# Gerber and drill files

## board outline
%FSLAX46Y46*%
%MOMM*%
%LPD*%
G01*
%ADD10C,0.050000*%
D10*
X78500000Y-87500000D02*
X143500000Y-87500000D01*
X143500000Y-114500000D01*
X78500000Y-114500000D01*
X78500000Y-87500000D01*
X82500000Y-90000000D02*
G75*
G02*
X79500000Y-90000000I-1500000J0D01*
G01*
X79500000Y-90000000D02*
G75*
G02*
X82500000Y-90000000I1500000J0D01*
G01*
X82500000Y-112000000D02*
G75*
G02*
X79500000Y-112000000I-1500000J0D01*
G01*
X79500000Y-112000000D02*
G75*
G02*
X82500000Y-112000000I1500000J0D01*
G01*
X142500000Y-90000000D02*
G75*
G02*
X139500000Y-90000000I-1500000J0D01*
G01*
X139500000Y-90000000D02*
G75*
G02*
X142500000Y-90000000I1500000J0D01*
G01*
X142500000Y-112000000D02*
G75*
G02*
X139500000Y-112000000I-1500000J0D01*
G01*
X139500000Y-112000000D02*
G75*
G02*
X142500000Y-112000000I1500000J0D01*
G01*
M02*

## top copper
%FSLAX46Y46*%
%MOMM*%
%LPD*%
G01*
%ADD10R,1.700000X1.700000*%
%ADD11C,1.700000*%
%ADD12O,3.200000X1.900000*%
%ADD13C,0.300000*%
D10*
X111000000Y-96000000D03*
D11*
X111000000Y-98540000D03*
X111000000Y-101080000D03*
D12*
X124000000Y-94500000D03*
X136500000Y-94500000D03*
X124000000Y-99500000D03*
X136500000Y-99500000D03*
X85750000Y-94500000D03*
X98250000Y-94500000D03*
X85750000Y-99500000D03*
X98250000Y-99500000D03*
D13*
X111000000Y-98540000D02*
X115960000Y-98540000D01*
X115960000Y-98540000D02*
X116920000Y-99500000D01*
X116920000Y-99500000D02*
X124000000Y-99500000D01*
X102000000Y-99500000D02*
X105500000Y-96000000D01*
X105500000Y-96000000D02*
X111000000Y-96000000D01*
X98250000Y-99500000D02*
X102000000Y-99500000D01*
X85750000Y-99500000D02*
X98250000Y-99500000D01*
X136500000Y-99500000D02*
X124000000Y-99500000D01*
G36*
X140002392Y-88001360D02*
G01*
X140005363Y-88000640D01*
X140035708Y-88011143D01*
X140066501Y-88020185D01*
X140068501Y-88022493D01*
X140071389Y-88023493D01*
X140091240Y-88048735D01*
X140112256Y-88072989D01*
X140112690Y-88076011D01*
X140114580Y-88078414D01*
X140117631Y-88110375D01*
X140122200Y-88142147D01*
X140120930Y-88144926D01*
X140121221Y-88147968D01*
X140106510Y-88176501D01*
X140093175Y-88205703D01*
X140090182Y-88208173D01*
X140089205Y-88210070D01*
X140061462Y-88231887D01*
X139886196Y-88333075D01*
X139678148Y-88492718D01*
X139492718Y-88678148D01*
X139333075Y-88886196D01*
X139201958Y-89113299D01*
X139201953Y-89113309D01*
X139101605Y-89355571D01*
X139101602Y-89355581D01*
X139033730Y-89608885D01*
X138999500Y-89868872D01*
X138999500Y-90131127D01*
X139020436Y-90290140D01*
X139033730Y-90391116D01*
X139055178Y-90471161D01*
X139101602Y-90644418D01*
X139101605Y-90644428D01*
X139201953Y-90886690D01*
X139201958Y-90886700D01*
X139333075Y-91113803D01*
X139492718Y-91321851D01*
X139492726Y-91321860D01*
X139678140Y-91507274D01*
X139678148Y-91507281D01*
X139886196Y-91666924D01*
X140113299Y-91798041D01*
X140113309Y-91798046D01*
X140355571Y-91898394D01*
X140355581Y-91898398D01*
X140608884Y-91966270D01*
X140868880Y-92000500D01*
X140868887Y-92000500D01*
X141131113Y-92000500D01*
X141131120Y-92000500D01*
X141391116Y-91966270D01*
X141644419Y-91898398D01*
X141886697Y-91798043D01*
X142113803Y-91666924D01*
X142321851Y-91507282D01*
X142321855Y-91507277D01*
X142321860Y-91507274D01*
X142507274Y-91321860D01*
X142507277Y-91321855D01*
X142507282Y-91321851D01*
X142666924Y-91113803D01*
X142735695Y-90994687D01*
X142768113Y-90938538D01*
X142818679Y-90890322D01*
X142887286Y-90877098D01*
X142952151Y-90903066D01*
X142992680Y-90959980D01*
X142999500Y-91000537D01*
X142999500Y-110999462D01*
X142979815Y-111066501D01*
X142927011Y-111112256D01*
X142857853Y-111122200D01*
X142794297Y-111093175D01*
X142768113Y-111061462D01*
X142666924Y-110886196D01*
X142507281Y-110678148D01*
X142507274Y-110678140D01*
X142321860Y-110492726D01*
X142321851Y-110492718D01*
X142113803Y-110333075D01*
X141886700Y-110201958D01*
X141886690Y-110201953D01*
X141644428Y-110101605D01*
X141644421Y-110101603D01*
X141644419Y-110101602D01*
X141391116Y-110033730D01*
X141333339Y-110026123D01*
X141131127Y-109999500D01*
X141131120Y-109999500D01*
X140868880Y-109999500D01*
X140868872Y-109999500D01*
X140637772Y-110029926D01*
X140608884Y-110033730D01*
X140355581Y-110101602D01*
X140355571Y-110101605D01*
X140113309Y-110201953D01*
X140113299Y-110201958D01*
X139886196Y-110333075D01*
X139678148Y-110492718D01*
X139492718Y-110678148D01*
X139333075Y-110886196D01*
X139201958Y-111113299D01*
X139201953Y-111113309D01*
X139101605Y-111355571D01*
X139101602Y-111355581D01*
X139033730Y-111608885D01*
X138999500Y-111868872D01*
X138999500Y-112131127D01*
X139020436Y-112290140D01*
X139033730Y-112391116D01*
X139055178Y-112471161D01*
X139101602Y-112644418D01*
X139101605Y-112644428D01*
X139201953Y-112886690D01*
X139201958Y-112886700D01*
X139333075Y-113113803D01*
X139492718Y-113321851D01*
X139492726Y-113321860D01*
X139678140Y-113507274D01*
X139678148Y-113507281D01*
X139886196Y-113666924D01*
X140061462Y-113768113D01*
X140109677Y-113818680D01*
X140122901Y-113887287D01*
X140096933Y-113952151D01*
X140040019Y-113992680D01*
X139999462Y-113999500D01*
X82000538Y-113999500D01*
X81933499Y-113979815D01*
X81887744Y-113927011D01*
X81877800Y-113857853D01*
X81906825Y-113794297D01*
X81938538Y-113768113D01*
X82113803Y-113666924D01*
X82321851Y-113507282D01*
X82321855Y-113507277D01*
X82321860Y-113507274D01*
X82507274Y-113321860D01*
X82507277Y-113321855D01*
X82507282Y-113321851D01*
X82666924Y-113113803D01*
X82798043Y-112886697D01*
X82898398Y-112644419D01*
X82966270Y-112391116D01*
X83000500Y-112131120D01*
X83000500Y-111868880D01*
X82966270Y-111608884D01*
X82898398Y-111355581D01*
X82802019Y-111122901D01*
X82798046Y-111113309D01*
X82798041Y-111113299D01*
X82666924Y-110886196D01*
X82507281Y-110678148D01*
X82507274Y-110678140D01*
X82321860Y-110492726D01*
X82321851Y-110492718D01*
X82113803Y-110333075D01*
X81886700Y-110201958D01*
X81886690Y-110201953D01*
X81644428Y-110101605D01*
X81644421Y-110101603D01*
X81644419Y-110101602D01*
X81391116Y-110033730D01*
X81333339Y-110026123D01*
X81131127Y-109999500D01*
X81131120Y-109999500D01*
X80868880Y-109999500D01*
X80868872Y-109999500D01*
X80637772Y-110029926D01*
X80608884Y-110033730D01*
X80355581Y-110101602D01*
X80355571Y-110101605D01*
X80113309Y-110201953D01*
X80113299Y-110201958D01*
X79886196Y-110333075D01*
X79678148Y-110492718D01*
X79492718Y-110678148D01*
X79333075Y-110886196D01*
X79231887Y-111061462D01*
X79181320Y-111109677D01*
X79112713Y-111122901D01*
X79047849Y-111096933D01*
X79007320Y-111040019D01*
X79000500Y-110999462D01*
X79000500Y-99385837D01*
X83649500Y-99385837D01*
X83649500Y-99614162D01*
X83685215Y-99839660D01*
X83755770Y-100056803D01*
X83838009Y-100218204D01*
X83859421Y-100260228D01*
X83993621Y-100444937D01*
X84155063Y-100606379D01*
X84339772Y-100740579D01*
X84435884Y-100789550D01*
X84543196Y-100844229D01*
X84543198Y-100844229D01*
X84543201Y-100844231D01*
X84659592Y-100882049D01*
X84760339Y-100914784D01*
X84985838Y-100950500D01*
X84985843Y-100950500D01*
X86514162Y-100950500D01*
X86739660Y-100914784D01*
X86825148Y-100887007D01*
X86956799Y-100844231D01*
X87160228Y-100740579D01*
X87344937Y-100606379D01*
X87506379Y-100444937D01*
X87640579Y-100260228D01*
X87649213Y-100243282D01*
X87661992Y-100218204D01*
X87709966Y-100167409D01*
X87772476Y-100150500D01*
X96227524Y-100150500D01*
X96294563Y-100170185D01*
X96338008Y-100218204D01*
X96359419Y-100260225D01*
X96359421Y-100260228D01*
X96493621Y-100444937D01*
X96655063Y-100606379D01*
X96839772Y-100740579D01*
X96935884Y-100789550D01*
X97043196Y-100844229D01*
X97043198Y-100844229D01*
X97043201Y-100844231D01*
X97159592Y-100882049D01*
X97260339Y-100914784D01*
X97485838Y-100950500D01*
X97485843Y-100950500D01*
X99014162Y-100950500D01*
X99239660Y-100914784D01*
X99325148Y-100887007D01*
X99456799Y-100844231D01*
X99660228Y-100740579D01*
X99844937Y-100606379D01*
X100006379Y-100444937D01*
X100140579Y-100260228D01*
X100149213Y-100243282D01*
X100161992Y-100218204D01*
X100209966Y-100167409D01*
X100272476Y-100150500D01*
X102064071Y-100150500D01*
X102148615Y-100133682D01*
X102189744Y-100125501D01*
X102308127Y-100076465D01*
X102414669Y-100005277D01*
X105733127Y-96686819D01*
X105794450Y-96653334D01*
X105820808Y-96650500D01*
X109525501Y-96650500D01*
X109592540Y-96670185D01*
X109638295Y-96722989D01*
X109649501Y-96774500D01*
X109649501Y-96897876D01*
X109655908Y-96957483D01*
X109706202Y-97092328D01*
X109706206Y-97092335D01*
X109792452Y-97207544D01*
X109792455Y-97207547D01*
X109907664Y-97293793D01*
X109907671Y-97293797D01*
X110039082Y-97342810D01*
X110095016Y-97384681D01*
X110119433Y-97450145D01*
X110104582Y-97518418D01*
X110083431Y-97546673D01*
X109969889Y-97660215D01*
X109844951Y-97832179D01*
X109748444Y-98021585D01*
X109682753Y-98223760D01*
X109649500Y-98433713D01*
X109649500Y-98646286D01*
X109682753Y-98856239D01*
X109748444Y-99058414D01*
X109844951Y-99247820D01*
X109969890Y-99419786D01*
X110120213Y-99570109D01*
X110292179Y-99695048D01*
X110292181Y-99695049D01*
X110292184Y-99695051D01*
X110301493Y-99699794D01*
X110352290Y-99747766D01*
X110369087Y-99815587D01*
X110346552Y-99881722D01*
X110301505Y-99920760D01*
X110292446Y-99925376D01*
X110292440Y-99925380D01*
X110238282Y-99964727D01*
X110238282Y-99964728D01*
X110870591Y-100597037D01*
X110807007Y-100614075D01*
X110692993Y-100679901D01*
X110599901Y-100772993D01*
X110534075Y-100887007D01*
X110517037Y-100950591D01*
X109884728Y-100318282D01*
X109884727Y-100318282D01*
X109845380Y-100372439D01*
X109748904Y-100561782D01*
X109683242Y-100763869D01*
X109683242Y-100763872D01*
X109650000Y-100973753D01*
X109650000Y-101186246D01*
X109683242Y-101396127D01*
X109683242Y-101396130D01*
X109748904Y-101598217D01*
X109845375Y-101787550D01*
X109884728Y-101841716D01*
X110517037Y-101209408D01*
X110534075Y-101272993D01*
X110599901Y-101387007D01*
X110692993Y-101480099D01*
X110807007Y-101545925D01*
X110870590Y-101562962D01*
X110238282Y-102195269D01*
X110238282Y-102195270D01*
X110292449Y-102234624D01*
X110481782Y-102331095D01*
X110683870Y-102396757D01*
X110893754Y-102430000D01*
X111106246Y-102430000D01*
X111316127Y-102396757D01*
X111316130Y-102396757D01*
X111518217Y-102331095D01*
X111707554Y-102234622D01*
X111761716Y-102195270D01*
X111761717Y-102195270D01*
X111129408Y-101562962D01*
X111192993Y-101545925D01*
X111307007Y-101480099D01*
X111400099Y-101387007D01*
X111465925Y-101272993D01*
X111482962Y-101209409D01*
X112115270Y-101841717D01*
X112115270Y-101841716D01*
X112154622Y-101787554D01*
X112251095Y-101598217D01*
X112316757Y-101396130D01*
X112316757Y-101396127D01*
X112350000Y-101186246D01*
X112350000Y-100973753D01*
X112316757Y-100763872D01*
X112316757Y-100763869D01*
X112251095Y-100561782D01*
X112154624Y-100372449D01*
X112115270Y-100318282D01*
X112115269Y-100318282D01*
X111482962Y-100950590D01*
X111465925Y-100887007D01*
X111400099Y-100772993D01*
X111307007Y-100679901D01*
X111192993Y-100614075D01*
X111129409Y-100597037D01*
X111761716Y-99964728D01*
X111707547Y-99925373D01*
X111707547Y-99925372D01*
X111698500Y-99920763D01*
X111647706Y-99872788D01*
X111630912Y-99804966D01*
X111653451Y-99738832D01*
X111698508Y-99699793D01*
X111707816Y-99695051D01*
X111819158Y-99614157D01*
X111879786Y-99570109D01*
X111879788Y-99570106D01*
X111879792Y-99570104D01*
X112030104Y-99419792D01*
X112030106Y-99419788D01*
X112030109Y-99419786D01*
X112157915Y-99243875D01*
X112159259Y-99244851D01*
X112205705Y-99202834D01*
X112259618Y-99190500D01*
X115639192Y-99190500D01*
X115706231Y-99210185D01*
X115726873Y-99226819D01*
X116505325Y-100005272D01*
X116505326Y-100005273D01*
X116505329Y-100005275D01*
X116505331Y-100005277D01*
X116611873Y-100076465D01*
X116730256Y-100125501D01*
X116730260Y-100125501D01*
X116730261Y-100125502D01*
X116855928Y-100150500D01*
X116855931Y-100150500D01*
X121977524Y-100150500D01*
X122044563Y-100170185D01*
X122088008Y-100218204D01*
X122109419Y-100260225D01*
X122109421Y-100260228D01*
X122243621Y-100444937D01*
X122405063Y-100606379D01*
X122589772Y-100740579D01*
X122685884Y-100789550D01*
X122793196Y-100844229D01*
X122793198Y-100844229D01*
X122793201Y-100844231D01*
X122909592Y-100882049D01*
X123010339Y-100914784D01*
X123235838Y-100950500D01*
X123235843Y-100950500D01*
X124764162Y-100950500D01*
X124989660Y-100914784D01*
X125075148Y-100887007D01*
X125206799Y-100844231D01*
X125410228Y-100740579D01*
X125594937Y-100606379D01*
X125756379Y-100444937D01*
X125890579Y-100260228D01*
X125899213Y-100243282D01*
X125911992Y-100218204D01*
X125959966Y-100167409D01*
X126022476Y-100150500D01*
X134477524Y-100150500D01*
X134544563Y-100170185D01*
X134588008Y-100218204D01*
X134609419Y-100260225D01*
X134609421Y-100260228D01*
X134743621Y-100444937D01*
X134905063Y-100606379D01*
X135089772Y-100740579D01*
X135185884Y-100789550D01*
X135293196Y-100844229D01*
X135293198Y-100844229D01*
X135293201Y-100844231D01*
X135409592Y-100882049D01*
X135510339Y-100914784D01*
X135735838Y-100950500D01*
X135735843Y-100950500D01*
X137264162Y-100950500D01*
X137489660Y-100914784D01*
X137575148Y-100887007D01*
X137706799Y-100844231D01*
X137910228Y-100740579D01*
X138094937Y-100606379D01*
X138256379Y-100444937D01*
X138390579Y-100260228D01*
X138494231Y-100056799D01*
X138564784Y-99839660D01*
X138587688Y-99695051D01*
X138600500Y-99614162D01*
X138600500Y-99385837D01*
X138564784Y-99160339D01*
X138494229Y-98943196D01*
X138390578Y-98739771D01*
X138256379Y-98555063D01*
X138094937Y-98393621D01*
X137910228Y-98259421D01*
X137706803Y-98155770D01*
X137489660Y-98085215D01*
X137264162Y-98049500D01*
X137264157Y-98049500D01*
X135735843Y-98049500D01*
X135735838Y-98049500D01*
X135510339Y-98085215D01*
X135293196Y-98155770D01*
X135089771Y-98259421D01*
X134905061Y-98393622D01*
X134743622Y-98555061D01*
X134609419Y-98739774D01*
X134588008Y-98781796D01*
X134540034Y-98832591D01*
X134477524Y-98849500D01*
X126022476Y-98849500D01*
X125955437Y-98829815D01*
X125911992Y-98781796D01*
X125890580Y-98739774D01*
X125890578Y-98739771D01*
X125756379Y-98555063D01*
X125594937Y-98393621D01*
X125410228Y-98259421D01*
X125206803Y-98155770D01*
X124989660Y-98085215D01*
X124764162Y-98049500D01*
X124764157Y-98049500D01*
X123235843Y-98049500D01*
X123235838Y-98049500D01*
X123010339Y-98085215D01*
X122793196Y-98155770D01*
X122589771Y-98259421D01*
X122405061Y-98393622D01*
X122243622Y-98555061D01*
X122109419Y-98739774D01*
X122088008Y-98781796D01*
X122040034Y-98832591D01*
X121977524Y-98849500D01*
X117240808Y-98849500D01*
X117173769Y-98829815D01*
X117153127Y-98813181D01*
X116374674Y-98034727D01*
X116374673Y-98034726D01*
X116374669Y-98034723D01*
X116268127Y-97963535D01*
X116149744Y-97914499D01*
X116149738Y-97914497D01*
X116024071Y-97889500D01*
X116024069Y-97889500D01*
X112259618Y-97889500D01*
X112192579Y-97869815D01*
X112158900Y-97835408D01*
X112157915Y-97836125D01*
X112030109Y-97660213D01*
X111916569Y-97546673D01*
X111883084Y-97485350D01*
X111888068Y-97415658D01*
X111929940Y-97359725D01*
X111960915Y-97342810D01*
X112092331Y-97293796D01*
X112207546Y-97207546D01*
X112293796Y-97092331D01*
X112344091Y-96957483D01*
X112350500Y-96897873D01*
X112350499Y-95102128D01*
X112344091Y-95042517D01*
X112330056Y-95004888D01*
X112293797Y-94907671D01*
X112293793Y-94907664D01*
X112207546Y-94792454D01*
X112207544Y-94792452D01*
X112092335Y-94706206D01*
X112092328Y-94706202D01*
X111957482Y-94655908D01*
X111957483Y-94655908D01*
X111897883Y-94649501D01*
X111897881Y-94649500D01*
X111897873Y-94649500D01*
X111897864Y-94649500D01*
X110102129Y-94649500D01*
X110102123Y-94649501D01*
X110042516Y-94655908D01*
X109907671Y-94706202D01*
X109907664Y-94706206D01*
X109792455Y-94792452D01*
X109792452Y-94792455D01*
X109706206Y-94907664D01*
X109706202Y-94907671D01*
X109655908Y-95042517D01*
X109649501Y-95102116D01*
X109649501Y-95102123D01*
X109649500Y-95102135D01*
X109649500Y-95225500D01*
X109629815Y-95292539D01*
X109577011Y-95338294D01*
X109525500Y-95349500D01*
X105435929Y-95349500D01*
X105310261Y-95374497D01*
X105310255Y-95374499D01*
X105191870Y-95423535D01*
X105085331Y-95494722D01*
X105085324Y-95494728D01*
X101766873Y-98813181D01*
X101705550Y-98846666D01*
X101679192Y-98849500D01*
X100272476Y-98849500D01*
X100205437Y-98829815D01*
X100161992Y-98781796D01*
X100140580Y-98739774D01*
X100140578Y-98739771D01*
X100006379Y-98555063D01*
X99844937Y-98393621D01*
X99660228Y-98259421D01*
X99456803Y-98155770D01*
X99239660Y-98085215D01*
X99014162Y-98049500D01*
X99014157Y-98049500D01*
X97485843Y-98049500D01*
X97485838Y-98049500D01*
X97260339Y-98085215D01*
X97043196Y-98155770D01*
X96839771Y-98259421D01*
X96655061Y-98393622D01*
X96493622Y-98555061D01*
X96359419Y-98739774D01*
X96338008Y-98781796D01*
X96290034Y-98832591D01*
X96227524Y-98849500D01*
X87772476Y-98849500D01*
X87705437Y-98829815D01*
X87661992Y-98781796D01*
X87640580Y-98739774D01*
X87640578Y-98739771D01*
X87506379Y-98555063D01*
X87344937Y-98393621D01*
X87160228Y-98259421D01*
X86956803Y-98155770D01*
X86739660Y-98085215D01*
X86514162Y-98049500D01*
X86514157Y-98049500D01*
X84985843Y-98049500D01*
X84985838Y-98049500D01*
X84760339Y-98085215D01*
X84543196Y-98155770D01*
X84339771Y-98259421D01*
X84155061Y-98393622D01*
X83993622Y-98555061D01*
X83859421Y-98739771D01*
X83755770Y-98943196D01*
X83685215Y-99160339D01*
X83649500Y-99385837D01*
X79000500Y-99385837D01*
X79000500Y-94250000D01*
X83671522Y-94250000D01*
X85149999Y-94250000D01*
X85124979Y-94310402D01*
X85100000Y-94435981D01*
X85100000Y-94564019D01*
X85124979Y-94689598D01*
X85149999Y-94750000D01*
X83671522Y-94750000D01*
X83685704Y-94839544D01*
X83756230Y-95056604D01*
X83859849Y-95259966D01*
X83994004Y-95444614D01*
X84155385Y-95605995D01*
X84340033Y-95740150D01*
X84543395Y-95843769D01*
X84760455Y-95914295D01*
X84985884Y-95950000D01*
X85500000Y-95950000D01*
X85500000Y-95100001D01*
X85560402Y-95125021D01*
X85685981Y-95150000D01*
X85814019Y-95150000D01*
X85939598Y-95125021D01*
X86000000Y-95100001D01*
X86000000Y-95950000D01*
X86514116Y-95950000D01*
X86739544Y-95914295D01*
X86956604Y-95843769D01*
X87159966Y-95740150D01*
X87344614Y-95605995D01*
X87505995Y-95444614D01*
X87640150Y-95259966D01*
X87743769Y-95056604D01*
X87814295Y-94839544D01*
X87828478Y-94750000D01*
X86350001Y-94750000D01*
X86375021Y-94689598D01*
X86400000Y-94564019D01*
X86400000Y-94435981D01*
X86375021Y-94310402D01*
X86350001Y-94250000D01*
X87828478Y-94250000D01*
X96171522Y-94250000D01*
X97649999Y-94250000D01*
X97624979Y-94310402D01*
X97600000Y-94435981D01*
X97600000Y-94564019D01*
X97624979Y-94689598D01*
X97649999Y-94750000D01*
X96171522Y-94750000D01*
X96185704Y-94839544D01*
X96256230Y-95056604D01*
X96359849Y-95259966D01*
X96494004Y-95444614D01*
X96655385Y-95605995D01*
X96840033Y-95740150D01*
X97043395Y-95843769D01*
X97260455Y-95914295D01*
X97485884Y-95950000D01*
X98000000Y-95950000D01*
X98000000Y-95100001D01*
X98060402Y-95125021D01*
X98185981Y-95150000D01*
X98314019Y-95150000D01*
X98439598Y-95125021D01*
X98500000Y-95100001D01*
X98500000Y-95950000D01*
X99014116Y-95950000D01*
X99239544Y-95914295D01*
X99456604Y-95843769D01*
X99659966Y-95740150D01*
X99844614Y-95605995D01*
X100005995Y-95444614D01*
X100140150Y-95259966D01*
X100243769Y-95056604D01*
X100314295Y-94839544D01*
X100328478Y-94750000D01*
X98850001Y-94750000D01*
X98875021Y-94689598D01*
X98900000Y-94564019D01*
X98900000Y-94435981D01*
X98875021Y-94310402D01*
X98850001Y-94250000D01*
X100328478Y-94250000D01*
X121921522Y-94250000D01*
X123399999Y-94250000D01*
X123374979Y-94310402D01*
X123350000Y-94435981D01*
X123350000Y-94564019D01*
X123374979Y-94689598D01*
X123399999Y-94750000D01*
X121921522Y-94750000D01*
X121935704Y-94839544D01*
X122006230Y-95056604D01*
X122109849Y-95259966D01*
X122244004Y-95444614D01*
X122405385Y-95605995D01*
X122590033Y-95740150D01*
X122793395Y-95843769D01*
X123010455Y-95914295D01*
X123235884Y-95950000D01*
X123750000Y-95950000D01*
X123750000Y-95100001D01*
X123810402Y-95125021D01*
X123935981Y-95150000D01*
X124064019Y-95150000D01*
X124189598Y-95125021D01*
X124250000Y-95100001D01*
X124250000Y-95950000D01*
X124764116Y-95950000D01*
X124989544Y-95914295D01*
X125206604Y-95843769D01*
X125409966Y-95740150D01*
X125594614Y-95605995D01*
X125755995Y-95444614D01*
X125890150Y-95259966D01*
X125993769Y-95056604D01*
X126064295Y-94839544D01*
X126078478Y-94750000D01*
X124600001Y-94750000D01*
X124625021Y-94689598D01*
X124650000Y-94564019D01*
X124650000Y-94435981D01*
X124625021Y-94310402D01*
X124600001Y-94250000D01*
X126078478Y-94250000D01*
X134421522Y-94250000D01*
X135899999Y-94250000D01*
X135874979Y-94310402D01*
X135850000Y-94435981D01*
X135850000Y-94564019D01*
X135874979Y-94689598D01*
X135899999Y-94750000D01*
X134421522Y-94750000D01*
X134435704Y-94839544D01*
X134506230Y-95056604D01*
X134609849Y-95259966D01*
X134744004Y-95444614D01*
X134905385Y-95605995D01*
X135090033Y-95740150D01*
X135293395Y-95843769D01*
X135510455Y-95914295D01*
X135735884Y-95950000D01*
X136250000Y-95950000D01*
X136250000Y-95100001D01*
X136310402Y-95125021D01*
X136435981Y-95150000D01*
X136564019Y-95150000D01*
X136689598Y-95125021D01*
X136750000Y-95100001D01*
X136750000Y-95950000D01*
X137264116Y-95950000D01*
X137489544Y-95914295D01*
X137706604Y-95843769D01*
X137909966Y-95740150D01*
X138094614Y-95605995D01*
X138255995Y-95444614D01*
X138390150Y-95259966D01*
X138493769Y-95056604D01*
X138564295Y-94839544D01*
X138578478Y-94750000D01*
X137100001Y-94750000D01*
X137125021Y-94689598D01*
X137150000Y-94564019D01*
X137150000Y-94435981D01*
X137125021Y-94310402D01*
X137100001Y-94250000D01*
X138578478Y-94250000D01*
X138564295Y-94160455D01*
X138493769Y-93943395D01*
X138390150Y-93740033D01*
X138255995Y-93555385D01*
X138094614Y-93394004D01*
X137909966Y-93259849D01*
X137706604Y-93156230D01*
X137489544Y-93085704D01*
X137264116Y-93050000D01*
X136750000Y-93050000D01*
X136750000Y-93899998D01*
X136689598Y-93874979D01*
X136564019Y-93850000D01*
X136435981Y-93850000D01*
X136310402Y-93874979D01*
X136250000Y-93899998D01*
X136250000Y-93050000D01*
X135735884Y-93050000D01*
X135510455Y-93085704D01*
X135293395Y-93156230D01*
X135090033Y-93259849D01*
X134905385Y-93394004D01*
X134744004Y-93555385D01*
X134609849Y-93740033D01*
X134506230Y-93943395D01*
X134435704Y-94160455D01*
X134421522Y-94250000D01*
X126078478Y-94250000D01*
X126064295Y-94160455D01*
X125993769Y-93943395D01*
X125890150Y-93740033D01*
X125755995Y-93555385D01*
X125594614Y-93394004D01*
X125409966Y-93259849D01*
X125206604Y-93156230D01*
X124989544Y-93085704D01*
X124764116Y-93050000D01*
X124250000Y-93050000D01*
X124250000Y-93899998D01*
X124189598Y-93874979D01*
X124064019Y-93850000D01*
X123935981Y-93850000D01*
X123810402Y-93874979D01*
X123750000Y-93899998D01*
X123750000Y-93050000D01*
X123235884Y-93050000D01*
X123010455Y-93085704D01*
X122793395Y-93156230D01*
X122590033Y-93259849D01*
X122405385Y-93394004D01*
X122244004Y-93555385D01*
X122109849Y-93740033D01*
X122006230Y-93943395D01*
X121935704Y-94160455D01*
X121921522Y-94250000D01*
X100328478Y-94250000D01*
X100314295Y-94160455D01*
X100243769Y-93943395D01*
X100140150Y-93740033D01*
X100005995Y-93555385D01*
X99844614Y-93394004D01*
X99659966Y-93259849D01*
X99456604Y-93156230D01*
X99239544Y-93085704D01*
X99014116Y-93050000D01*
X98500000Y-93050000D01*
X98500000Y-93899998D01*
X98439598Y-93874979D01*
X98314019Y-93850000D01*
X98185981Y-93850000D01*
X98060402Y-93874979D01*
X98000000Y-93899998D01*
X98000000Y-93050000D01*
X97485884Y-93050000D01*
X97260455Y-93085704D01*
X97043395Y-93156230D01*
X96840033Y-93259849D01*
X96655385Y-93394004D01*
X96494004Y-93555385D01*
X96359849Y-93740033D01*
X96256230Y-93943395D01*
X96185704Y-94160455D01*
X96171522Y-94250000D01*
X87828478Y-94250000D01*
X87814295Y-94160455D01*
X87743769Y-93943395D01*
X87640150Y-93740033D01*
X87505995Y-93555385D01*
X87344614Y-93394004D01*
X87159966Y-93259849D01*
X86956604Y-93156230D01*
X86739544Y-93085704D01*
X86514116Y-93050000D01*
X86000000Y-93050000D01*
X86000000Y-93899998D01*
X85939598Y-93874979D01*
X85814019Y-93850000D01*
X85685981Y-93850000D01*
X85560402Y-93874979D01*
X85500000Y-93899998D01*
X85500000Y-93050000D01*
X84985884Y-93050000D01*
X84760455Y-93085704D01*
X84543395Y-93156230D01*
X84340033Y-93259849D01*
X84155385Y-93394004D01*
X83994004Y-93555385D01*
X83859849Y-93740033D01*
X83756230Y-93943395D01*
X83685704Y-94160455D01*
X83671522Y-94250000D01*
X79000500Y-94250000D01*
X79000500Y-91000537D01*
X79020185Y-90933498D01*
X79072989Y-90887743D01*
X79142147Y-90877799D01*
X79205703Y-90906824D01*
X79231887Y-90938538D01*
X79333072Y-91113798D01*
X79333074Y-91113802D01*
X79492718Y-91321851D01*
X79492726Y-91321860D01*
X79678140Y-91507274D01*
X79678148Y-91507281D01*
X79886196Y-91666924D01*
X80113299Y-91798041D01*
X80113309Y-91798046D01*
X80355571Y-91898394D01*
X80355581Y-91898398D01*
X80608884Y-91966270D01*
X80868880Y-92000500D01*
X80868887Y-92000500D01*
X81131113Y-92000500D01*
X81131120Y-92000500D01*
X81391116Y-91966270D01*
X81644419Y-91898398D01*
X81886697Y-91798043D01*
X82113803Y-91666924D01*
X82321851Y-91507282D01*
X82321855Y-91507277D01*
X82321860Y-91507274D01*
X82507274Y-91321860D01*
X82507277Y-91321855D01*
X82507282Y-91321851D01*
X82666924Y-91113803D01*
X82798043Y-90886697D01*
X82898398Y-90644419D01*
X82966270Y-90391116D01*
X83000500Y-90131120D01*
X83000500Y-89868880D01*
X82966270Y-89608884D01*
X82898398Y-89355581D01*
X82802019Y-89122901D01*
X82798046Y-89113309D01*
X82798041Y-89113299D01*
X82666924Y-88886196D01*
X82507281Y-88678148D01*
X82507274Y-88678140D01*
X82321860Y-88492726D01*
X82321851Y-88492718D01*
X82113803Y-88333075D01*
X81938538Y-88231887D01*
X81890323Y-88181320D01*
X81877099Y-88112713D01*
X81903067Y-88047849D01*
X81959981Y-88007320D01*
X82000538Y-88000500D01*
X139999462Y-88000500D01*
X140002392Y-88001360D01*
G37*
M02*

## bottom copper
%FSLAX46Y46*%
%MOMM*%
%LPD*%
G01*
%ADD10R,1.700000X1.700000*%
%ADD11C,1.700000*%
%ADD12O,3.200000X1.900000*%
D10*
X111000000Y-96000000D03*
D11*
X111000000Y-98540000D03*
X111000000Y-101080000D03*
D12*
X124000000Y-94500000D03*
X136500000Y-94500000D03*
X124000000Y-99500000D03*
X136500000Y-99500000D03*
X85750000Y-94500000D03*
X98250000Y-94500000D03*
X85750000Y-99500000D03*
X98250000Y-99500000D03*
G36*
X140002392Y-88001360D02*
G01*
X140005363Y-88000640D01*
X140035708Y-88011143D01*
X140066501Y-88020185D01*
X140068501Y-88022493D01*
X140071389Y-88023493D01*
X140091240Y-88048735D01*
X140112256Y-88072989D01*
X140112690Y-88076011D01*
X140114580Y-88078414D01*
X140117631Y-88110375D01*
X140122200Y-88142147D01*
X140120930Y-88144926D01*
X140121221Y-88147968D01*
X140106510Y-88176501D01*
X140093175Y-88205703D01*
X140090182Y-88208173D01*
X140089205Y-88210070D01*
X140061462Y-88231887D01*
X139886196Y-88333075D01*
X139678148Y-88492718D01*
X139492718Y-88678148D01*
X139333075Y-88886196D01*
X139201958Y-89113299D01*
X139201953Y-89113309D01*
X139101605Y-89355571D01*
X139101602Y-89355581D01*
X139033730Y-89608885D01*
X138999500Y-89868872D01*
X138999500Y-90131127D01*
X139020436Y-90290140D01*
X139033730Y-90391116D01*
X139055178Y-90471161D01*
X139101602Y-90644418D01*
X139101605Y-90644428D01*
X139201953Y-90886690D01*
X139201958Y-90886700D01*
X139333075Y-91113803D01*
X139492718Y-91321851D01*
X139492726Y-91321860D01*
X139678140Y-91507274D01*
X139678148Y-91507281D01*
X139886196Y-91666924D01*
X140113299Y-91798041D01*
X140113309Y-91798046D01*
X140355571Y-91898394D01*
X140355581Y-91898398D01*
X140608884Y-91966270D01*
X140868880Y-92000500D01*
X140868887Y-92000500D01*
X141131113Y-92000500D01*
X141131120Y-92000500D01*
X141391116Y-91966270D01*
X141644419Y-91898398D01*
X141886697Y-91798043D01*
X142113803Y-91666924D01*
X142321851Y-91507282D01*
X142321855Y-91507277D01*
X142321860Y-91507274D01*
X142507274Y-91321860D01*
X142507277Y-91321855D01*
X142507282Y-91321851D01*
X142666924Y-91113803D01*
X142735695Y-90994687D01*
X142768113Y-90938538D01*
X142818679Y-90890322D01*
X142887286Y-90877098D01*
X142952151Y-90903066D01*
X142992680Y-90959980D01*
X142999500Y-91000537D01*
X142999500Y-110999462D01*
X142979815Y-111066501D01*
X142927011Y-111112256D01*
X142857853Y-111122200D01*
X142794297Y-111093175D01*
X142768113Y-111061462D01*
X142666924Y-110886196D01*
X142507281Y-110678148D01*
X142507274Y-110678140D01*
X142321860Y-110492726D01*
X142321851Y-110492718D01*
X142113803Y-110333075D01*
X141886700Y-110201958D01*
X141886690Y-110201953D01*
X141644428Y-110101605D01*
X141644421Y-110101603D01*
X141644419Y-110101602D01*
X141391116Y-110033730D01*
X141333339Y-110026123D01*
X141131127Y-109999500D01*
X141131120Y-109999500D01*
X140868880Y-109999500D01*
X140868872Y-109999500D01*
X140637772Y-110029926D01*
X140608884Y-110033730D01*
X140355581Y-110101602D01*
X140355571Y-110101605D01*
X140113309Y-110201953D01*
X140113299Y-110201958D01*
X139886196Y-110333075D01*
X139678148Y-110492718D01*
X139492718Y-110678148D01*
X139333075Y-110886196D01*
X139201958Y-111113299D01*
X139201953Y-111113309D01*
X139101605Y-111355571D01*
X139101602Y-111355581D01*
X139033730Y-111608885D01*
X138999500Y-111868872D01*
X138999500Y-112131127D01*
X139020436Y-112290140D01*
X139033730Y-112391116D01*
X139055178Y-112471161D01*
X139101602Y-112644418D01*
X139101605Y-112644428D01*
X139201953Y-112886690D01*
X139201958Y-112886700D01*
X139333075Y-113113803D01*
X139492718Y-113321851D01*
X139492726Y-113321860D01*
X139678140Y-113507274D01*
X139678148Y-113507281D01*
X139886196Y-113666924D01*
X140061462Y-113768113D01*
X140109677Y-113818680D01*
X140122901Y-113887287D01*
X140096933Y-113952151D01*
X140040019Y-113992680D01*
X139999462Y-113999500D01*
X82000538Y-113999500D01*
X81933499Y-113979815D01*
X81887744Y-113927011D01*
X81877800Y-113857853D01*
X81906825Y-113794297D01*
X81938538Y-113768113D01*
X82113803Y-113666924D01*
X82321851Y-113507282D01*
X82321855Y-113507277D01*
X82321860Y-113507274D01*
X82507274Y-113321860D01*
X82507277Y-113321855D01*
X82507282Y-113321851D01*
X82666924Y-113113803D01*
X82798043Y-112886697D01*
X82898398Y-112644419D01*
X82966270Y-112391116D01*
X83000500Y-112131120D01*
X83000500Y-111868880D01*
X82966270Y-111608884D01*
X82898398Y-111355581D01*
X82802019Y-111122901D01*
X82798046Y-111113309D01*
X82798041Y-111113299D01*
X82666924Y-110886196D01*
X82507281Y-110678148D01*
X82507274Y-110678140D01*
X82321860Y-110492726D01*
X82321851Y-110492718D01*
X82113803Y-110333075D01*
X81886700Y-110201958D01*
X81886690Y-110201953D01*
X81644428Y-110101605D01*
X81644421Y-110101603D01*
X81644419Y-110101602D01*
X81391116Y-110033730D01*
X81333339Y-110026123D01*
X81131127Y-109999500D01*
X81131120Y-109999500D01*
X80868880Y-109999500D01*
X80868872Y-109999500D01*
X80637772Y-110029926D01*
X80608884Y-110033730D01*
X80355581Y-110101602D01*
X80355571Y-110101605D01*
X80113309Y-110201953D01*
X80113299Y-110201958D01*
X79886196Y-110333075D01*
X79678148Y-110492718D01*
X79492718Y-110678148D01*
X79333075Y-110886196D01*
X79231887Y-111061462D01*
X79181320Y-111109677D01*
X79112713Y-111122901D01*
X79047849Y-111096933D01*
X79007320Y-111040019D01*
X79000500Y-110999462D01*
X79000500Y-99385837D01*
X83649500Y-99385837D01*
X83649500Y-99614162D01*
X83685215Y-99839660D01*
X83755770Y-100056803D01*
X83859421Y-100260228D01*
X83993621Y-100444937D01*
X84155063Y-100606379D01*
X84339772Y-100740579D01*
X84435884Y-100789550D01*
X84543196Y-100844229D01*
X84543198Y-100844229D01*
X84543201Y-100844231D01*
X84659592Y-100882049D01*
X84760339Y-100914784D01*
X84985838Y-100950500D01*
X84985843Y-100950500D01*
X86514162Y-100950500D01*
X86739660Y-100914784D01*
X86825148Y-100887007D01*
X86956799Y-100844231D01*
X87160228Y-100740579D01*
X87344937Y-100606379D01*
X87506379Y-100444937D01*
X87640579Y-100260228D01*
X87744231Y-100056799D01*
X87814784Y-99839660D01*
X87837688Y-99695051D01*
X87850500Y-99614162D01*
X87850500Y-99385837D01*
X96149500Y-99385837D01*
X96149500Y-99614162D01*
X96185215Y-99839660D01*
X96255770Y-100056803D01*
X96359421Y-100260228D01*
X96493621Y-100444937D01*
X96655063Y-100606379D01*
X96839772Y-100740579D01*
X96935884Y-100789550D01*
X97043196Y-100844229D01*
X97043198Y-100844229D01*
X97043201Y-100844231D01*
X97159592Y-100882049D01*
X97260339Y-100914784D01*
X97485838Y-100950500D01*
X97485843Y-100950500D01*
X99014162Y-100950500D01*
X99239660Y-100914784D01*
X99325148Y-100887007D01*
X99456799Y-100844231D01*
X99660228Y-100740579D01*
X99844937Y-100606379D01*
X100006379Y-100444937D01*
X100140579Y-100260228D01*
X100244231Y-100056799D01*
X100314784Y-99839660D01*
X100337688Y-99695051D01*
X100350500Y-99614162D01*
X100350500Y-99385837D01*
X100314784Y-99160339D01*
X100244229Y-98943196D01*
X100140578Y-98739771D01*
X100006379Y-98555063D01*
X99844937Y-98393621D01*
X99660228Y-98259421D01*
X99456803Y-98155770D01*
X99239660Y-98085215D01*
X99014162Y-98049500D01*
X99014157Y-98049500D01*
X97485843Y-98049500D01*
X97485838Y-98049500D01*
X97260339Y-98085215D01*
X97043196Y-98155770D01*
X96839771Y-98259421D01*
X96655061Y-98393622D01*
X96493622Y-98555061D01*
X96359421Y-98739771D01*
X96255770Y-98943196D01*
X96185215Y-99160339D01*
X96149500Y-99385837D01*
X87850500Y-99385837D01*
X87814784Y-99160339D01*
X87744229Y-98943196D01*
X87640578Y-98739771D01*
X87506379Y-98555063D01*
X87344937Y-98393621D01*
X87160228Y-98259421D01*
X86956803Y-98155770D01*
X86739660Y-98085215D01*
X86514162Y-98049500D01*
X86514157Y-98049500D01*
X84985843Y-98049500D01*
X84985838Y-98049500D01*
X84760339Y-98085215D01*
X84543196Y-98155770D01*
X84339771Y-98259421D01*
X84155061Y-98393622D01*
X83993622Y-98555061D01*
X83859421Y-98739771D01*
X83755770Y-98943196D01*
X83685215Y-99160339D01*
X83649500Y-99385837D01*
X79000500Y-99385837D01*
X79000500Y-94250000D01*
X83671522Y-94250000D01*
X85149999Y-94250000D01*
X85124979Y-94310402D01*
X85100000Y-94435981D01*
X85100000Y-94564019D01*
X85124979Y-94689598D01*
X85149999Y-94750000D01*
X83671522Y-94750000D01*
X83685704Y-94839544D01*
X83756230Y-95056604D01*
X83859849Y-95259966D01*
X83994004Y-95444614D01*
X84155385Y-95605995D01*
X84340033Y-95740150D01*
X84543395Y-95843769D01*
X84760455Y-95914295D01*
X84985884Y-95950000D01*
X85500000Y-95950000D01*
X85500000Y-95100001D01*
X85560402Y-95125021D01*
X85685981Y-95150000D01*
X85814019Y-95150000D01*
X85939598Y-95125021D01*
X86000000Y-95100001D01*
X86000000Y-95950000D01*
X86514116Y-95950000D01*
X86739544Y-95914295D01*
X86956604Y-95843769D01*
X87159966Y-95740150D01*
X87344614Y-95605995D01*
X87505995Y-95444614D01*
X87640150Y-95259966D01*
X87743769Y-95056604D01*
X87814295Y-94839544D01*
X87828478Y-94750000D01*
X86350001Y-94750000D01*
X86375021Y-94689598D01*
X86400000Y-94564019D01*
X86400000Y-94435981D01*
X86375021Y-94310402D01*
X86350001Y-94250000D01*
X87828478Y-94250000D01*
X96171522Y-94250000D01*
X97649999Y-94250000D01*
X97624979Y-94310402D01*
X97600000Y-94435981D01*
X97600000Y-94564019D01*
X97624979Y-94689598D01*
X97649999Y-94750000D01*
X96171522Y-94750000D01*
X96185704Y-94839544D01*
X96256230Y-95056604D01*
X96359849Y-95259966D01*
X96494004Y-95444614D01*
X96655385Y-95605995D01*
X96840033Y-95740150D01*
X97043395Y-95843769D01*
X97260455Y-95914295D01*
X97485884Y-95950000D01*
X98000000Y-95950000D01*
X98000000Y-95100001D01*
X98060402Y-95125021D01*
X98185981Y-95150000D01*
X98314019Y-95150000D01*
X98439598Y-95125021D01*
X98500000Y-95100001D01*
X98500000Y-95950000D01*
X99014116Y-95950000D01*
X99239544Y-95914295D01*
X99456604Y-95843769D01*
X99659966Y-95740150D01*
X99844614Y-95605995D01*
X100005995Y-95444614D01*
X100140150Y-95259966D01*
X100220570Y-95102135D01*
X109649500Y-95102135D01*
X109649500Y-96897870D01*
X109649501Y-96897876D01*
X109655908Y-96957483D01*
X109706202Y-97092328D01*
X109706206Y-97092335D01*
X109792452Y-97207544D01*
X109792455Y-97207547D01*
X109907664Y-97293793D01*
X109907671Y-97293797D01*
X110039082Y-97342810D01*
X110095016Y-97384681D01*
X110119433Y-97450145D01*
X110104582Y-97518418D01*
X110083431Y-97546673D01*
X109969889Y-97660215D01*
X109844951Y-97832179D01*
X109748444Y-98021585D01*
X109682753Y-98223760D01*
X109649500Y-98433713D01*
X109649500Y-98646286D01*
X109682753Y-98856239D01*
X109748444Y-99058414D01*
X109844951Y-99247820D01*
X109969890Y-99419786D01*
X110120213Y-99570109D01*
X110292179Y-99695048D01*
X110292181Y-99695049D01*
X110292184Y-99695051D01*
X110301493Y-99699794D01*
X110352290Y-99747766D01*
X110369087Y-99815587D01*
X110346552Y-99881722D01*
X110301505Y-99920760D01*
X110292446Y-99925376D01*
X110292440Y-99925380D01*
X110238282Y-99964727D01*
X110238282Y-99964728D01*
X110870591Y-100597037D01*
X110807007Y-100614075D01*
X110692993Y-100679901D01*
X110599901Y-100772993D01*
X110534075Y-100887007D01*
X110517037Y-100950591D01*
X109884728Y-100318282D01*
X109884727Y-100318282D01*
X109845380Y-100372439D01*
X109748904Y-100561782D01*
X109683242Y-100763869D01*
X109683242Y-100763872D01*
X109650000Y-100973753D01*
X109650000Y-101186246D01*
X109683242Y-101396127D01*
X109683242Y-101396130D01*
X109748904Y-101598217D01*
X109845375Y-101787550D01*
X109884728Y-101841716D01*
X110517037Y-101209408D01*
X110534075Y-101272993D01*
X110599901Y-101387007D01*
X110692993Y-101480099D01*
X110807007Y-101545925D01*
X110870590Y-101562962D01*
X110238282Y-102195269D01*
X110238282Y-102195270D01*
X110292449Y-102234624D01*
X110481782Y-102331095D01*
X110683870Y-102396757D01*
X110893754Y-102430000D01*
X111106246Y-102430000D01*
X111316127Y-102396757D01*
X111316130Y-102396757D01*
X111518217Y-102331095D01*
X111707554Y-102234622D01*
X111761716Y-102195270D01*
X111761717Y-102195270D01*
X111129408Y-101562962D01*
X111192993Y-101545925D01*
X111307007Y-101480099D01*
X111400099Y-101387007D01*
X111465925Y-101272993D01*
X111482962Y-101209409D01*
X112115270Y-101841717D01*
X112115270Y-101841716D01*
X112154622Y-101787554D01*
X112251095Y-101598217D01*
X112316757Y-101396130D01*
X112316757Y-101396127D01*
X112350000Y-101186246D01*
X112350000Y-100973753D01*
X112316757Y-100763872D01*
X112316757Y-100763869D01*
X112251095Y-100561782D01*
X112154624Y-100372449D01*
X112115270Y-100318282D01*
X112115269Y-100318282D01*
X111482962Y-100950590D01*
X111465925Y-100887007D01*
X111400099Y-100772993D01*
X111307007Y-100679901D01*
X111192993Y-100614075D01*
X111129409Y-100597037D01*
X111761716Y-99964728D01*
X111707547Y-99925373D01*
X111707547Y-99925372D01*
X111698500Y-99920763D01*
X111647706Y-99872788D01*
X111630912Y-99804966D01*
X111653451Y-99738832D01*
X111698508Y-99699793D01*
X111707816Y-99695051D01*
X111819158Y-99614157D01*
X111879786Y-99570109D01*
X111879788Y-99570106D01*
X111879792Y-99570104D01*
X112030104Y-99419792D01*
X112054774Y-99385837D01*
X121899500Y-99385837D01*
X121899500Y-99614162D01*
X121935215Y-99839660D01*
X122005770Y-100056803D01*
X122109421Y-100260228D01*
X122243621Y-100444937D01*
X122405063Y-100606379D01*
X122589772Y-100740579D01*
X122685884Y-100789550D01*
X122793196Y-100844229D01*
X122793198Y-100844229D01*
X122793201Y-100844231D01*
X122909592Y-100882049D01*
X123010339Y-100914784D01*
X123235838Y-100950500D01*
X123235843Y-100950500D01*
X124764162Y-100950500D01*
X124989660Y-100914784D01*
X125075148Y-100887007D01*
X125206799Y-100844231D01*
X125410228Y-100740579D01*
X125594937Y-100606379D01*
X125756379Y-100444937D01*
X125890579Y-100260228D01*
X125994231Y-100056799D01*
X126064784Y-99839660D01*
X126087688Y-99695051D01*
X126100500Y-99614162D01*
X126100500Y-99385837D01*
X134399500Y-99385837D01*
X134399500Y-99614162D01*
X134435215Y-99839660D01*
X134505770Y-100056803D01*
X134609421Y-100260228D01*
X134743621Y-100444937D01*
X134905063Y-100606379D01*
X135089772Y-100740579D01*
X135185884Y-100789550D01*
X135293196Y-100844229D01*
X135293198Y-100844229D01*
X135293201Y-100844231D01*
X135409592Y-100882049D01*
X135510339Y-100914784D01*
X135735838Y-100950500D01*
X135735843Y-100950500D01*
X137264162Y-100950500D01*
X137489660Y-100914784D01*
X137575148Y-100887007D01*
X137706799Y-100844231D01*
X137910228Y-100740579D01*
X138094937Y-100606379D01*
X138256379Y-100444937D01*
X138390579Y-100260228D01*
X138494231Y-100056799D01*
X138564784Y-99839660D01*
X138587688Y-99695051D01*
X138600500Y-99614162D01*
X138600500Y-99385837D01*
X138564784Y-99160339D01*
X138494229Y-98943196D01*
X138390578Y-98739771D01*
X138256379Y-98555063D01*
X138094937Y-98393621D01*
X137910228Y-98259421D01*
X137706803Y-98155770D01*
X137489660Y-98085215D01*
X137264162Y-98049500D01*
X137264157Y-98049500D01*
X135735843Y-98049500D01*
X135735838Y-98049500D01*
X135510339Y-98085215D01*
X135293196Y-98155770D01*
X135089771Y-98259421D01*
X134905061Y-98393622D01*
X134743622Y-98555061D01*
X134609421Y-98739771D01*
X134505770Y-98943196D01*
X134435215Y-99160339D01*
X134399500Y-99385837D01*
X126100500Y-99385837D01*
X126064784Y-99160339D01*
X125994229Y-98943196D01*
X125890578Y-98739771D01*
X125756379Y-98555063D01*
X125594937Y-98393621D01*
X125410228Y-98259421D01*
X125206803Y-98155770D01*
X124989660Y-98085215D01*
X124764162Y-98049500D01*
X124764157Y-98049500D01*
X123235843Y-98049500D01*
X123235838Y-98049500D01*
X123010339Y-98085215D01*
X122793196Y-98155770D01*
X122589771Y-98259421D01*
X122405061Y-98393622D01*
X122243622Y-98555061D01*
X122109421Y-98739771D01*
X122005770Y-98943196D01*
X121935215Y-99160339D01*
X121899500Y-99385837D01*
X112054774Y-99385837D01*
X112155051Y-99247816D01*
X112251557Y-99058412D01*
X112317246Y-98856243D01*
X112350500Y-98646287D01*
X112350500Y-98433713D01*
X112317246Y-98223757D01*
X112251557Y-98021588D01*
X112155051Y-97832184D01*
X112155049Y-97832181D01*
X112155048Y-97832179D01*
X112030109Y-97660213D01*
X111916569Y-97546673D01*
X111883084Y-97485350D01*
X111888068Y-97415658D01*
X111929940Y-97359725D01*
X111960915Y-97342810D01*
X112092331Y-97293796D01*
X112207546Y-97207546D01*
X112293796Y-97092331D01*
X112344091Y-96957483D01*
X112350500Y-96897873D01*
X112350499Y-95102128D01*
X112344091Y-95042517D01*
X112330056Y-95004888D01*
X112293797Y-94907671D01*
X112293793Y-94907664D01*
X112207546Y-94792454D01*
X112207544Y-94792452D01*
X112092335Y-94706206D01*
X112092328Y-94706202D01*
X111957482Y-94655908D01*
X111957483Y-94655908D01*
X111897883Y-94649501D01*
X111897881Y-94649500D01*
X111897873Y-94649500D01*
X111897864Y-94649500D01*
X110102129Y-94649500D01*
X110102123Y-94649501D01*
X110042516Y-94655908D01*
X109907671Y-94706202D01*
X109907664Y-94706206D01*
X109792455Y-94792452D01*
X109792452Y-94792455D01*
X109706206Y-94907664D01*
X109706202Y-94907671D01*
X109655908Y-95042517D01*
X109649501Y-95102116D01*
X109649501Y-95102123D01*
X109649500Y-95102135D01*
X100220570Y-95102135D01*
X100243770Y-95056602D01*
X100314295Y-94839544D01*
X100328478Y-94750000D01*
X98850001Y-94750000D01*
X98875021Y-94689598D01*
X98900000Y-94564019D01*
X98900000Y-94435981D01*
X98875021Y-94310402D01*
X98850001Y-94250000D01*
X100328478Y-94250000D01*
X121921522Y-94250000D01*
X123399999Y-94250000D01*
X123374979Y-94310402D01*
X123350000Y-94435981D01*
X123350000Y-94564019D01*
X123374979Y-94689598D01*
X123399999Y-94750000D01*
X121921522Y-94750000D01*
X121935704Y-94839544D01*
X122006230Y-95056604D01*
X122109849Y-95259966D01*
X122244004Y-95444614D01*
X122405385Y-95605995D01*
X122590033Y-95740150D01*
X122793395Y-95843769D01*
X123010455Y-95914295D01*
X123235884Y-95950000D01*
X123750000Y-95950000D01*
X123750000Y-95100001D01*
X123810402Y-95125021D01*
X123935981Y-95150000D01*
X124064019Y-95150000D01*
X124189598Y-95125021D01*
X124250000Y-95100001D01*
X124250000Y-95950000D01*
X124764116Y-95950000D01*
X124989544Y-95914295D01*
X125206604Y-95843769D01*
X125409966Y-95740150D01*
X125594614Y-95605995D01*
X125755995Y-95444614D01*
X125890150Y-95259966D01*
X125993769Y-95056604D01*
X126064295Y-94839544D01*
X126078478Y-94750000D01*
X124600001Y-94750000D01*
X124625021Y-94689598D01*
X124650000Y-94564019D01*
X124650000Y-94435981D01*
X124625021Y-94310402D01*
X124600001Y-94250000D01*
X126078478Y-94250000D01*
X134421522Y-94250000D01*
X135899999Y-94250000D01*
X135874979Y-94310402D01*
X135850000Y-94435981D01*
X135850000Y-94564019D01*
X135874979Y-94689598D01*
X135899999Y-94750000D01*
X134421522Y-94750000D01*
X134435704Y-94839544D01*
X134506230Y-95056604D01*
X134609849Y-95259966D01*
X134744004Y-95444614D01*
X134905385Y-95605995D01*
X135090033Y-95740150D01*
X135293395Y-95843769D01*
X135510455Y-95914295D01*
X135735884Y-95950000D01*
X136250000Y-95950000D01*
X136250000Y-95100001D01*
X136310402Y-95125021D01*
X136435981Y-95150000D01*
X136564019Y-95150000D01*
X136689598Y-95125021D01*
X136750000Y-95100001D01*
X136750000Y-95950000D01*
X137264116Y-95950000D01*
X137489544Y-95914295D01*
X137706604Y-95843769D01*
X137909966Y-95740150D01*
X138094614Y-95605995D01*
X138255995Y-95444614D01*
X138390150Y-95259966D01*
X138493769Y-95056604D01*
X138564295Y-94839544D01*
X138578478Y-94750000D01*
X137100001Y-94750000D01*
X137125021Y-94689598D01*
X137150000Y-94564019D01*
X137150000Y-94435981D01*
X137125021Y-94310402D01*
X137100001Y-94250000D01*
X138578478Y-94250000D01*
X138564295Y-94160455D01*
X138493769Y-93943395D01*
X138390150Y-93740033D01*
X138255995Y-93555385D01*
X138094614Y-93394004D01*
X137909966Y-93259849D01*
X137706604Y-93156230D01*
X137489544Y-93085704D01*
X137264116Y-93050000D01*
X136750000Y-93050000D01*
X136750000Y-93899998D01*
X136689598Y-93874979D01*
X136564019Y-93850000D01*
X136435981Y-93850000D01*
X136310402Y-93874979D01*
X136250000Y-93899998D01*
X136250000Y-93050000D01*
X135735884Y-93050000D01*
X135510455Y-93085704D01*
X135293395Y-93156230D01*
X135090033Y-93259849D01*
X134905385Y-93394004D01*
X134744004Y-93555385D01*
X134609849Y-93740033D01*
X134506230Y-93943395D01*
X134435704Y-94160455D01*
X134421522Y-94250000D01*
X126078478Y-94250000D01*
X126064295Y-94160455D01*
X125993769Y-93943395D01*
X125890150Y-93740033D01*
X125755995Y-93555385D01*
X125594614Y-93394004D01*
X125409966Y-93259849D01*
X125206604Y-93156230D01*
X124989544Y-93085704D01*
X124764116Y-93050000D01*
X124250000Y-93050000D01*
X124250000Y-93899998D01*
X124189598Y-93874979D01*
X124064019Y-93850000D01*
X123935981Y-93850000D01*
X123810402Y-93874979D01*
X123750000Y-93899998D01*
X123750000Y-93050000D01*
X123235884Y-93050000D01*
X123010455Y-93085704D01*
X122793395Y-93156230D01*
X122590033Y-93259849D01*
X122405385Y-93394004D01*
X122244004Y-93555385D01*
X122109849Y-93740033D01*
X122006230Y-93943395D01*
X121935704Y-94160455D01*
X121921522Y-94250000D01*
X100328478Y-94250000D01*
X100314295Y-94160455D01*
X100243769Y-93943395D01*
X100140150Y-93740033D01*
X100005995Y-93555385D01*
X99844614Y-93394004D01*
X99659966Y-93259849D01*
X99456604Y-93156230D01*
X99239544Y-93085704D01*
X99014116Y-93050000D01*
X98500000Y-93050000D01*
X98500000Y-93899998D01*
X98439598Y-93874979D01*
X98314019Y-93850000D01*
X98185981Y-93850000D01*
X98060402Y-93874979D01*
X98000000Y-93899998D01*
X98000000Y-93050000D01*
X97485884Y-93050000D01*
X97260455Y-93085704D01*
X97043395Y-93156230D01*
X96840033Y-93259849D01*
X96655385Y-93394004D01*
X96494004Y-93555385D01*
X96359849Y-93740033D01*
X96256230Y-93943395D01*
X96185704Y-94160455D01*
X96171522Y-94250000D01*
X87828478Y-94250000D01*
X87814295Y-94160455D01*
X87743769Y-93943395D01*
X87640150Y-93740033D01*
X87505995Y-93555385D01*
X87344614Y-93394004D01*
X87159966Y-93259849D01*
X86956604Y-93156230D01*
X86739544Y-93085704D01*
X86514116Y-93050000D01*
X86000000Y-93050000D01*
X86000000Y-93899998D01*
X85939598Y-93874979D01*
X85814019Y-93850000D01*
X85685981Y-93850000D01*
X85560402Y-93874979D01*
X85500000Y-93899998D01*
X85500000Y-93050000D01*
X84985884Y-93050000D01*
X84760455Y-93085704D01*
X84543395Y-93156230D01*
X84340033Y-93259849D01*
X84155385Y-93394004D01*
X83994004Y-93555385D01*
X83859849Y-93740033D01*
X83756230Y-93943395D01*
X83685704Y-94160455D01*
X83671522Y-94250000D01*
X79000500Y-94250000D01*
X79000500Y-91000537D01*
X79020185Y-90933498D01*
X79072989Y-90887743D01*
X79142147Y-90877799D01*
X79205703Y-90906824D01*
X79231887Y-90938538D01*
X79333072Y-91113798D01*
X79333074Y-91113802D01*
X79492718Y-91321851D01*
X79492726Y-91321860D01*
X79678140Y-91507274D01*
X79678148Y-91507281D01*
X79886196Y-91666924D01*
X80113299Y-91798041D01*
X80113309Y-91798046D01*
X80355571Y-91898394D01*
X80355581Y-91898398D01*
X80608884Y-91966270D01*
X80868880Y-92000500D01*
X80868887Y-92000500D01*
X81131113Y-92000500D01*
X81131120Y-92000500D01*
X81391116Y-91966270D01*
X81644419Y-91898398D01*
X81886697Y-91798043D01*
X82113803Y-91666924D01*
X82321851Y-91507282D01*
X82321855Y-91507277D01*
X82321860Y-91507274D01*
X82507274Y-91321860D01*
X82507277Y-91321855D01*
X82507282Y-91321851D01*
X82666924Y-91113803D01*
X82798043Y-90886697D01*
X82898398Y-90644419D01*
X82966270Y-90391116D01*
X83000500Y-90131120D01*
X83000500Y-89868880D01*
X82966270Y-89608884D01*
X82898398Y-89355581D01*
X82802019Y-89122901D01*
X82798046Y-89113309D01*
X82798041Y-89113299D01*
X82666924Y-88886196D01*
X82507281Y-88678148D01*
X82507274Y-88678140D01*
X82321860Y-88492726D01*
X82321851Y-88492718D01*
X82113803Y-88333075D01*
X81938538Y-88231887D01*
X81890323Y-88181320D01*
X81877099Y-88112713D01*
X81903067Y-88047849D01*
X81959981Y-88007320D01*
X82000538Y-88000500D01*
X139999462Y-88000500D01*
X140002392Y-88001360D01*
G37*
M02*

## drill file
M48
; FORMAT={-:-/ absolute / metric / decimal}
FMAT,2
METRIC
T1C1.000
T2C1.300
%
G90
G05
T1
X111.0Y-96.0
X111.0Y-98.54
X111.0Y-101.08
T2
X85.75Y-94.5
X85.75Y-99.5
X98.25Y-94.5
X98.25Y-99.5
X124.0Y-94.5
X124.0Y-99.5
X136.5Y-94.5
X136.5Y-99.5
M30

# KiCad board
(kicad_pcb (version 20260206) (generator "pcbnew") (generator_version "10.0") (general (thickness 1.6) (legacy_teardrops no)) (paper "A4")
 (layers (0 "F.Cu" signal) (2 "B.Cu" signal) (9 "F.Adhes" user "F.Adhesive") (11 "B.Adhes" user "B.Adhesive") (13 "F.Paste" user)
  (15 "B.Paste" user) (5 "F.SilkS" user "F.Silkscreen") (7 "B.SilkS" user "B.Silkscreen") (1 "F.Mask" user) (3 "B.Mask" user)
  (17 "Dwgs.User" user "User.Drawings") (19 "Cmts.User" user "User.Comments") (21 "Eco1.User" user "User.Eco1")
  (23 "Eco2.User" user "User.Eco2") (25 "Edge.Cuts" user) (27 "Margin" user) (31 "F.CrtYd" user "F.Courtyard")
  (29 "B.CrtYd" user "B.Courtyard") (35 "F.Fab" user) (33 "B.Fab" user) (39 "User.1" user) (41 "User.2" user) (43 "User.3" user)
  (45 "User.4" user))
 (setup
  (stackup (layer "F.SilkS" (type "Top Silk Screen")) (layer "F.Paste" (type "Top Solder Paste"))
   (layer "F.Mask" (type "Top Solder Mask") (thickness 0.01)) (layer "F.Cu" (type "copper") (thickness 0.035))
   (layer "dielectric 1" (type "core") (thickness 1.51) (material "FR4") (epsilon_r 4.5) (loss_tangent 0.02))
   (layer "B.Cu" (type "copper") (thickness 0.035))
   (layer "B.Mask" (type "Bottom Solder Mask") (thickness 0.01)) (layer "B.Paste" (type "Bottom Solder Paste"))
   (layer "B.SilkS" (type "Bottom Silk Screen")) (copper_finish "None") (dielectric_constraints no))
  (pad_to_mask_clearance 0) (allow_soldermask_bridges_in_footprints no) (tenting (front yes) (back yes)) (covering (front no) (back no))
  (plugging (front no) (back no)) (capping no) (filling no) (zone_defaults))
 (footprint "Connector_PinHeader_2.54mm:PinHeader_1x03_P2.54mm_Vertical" (layer "F.Cu") (at 111 96)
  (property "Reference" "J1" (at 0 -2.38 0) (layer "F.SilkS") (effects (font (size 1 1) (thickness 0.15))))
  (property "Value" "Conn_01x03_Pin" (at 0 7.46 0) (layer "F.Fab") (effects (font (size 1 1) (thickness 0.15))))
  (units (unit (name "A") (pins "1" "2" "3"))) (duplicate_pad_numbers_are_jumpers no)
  (pad "1" thru_hole rect (at 0 0) (size 1.7 1.7) (drill 1) (layers "*.Cu" "*.Mask") (remove_unused_layers no) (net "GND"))
  (pad "2" thru_hole circle (at 0 2.54) (size 1.7 1.7) (drill 1) (layers "*.Cu" "*.Mask") (remove_unused_layers no) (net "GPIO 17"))
  (pad "3" thru_hole circle (at 0 5.08) (size 1.7 1.7) (drill 1) (layers "*.Cu" "*.Mask") (remove_unused_layers no) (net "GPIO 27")))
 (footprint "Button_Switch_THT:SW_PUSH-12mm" (layer "F.Cu") (at 124 94.5)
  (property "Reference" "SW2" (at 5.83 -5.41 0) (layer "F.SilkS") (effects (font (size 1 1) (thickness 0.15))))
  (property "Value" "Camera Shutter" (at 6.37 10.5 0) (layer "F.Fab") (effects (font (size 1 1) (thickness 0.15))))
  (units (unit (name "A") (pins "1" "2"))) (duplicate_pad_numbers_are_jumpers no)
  (pad "1" thru_hole oval (at 0 0) (size 3.2 1.9) (drill 1.3) (layers "*.Cu" "*.Mask") (remove_unused_layers no) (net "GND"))
  (pad "1" thru_hole oval (at 12.5 0) (size 3.2 1.9) (drill 1.3) (layers "*.Cu" "*.Mask") (remove_unused_layers no) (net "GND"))
  (pad "2" thru_hole oval (at 0 5) (size 3.2 1.9) (drill 1.3) (layers "*.Cu" "*.Mask") (remove_unused_layers no) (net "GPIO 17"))
  (pad "2" thru_hole oval (at 12.5 5) (size 3.2 1.9) (drill 1.3) (layers "*.Cu" "*.Mask") (remove_unused_layers no) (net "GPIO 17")))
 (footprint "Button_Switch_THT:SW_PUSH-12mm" (layer "F.Cu") (at 85.75 94.5)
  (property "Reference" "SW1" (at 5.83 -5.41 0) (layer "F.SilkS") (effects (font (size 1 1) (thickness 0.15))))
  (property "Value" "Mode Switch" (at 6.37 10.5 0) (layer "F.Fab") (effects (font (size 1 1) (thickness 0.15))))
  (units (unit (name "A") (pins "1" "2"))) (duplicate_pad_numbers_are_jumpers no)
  (pad "1" thru_hole oval (at 0 0) (size 3.2 1.9) (drill 1.3) (layers "*.Cu" "*.Mask") (remove_unused_layers no) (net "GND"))
  (pad "1" thru_hole oval (at 12.5 0) (size 3.2 1.9) (drill 1.3) (layers "*.Cu" "*.Mask") (remove_unused_layers no) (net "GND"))
  (pad "2" thru_hole oval (at 0 5) (size 3.2 1.9) (drill 1.3) (layers "*.Cu" "*.Mask") (remove_unused_layers no) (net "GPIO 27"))
  (pad "2" thru_hole oval (at 12.5 5) (size 3.2 1.9) (drill 1.3) (layers "*.Cu" "*.Mask") (remove_unused_layers no) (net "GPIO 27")))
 (gr_rect (start 78.5 87.5) (end 143.5 114.5) (stroke (width 0.05) (type solid)) (fill no) (layer "Edge.Cuts"))
 (gr_circle (center 81 90) (end 82.5 90) (stroke (width 0.05) (type solid)) (fill no) (layer "Edge.Cuts"))
 (gr_circle (center 81 112) (end 82.5 112) (stroke (width 0.05) (type solid)) (fill no) (layer "Edge.Cuts"))
 (gr_circle (center 141 90) (end 142.5 90) (stroke (width 0.05) (type solid)) (fill no) (layer "Edge.Cuts"))
 (gr_circle (center 141 112) (end 142.5 112) (stroke (width 0.05) (type solid)) (fill no) (layer "Edge.Cuts"))
 (segment (start 105.42 101.08) (end 111 101.08) (width 0.3) (layer "F.Cu") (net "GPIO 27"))
 (segment (start 103.5 99.5) (end 105.08 101.08) (width 0.3) (layer "F.Cu") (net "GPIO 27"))
 (segment (start 98.25 99.5) (end 103.5 99.5) (width 0.3) (layer "F.Cu") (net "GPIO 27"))
 (segment (start 85.75 99.5) (end 98.25 99.5) (width 0.3) (layer "F.Cu") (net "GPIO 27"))
 (segment (start 105.08 101.08) (end 105.42 101.08) (width 0.3) (layer "F.Cu") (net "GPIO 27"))
 (segment (start 115.96 98.54) (end 111 98.54) (width 0.3) (layer "F.Cu") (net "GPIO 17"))
 (segment (start 124 99.5) (end 117 99.5) (width 0.3) (layer "F.Cu") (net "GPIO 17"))
 (segment (start 116 98.5) (end 115.96 98.54) (width 0.3) (layer "F.Cu") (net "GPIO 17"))
 (segment (start 117 99.5) (end 116 98.5) (width 0.3) (layer "F.Cu") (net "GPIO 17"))
 (segment (start 136.5 99.5) (end 124 99.5) (width 0.3) (layer "F.Cu") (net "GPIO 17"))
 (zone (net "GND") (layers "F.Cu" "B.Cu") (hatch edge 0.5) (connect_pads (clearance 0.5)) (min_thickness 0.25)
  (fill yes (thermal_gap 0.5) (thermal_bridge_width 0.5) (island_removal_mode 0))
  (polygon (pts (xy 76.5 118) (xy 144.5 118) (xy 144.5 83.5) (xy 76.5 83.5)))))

